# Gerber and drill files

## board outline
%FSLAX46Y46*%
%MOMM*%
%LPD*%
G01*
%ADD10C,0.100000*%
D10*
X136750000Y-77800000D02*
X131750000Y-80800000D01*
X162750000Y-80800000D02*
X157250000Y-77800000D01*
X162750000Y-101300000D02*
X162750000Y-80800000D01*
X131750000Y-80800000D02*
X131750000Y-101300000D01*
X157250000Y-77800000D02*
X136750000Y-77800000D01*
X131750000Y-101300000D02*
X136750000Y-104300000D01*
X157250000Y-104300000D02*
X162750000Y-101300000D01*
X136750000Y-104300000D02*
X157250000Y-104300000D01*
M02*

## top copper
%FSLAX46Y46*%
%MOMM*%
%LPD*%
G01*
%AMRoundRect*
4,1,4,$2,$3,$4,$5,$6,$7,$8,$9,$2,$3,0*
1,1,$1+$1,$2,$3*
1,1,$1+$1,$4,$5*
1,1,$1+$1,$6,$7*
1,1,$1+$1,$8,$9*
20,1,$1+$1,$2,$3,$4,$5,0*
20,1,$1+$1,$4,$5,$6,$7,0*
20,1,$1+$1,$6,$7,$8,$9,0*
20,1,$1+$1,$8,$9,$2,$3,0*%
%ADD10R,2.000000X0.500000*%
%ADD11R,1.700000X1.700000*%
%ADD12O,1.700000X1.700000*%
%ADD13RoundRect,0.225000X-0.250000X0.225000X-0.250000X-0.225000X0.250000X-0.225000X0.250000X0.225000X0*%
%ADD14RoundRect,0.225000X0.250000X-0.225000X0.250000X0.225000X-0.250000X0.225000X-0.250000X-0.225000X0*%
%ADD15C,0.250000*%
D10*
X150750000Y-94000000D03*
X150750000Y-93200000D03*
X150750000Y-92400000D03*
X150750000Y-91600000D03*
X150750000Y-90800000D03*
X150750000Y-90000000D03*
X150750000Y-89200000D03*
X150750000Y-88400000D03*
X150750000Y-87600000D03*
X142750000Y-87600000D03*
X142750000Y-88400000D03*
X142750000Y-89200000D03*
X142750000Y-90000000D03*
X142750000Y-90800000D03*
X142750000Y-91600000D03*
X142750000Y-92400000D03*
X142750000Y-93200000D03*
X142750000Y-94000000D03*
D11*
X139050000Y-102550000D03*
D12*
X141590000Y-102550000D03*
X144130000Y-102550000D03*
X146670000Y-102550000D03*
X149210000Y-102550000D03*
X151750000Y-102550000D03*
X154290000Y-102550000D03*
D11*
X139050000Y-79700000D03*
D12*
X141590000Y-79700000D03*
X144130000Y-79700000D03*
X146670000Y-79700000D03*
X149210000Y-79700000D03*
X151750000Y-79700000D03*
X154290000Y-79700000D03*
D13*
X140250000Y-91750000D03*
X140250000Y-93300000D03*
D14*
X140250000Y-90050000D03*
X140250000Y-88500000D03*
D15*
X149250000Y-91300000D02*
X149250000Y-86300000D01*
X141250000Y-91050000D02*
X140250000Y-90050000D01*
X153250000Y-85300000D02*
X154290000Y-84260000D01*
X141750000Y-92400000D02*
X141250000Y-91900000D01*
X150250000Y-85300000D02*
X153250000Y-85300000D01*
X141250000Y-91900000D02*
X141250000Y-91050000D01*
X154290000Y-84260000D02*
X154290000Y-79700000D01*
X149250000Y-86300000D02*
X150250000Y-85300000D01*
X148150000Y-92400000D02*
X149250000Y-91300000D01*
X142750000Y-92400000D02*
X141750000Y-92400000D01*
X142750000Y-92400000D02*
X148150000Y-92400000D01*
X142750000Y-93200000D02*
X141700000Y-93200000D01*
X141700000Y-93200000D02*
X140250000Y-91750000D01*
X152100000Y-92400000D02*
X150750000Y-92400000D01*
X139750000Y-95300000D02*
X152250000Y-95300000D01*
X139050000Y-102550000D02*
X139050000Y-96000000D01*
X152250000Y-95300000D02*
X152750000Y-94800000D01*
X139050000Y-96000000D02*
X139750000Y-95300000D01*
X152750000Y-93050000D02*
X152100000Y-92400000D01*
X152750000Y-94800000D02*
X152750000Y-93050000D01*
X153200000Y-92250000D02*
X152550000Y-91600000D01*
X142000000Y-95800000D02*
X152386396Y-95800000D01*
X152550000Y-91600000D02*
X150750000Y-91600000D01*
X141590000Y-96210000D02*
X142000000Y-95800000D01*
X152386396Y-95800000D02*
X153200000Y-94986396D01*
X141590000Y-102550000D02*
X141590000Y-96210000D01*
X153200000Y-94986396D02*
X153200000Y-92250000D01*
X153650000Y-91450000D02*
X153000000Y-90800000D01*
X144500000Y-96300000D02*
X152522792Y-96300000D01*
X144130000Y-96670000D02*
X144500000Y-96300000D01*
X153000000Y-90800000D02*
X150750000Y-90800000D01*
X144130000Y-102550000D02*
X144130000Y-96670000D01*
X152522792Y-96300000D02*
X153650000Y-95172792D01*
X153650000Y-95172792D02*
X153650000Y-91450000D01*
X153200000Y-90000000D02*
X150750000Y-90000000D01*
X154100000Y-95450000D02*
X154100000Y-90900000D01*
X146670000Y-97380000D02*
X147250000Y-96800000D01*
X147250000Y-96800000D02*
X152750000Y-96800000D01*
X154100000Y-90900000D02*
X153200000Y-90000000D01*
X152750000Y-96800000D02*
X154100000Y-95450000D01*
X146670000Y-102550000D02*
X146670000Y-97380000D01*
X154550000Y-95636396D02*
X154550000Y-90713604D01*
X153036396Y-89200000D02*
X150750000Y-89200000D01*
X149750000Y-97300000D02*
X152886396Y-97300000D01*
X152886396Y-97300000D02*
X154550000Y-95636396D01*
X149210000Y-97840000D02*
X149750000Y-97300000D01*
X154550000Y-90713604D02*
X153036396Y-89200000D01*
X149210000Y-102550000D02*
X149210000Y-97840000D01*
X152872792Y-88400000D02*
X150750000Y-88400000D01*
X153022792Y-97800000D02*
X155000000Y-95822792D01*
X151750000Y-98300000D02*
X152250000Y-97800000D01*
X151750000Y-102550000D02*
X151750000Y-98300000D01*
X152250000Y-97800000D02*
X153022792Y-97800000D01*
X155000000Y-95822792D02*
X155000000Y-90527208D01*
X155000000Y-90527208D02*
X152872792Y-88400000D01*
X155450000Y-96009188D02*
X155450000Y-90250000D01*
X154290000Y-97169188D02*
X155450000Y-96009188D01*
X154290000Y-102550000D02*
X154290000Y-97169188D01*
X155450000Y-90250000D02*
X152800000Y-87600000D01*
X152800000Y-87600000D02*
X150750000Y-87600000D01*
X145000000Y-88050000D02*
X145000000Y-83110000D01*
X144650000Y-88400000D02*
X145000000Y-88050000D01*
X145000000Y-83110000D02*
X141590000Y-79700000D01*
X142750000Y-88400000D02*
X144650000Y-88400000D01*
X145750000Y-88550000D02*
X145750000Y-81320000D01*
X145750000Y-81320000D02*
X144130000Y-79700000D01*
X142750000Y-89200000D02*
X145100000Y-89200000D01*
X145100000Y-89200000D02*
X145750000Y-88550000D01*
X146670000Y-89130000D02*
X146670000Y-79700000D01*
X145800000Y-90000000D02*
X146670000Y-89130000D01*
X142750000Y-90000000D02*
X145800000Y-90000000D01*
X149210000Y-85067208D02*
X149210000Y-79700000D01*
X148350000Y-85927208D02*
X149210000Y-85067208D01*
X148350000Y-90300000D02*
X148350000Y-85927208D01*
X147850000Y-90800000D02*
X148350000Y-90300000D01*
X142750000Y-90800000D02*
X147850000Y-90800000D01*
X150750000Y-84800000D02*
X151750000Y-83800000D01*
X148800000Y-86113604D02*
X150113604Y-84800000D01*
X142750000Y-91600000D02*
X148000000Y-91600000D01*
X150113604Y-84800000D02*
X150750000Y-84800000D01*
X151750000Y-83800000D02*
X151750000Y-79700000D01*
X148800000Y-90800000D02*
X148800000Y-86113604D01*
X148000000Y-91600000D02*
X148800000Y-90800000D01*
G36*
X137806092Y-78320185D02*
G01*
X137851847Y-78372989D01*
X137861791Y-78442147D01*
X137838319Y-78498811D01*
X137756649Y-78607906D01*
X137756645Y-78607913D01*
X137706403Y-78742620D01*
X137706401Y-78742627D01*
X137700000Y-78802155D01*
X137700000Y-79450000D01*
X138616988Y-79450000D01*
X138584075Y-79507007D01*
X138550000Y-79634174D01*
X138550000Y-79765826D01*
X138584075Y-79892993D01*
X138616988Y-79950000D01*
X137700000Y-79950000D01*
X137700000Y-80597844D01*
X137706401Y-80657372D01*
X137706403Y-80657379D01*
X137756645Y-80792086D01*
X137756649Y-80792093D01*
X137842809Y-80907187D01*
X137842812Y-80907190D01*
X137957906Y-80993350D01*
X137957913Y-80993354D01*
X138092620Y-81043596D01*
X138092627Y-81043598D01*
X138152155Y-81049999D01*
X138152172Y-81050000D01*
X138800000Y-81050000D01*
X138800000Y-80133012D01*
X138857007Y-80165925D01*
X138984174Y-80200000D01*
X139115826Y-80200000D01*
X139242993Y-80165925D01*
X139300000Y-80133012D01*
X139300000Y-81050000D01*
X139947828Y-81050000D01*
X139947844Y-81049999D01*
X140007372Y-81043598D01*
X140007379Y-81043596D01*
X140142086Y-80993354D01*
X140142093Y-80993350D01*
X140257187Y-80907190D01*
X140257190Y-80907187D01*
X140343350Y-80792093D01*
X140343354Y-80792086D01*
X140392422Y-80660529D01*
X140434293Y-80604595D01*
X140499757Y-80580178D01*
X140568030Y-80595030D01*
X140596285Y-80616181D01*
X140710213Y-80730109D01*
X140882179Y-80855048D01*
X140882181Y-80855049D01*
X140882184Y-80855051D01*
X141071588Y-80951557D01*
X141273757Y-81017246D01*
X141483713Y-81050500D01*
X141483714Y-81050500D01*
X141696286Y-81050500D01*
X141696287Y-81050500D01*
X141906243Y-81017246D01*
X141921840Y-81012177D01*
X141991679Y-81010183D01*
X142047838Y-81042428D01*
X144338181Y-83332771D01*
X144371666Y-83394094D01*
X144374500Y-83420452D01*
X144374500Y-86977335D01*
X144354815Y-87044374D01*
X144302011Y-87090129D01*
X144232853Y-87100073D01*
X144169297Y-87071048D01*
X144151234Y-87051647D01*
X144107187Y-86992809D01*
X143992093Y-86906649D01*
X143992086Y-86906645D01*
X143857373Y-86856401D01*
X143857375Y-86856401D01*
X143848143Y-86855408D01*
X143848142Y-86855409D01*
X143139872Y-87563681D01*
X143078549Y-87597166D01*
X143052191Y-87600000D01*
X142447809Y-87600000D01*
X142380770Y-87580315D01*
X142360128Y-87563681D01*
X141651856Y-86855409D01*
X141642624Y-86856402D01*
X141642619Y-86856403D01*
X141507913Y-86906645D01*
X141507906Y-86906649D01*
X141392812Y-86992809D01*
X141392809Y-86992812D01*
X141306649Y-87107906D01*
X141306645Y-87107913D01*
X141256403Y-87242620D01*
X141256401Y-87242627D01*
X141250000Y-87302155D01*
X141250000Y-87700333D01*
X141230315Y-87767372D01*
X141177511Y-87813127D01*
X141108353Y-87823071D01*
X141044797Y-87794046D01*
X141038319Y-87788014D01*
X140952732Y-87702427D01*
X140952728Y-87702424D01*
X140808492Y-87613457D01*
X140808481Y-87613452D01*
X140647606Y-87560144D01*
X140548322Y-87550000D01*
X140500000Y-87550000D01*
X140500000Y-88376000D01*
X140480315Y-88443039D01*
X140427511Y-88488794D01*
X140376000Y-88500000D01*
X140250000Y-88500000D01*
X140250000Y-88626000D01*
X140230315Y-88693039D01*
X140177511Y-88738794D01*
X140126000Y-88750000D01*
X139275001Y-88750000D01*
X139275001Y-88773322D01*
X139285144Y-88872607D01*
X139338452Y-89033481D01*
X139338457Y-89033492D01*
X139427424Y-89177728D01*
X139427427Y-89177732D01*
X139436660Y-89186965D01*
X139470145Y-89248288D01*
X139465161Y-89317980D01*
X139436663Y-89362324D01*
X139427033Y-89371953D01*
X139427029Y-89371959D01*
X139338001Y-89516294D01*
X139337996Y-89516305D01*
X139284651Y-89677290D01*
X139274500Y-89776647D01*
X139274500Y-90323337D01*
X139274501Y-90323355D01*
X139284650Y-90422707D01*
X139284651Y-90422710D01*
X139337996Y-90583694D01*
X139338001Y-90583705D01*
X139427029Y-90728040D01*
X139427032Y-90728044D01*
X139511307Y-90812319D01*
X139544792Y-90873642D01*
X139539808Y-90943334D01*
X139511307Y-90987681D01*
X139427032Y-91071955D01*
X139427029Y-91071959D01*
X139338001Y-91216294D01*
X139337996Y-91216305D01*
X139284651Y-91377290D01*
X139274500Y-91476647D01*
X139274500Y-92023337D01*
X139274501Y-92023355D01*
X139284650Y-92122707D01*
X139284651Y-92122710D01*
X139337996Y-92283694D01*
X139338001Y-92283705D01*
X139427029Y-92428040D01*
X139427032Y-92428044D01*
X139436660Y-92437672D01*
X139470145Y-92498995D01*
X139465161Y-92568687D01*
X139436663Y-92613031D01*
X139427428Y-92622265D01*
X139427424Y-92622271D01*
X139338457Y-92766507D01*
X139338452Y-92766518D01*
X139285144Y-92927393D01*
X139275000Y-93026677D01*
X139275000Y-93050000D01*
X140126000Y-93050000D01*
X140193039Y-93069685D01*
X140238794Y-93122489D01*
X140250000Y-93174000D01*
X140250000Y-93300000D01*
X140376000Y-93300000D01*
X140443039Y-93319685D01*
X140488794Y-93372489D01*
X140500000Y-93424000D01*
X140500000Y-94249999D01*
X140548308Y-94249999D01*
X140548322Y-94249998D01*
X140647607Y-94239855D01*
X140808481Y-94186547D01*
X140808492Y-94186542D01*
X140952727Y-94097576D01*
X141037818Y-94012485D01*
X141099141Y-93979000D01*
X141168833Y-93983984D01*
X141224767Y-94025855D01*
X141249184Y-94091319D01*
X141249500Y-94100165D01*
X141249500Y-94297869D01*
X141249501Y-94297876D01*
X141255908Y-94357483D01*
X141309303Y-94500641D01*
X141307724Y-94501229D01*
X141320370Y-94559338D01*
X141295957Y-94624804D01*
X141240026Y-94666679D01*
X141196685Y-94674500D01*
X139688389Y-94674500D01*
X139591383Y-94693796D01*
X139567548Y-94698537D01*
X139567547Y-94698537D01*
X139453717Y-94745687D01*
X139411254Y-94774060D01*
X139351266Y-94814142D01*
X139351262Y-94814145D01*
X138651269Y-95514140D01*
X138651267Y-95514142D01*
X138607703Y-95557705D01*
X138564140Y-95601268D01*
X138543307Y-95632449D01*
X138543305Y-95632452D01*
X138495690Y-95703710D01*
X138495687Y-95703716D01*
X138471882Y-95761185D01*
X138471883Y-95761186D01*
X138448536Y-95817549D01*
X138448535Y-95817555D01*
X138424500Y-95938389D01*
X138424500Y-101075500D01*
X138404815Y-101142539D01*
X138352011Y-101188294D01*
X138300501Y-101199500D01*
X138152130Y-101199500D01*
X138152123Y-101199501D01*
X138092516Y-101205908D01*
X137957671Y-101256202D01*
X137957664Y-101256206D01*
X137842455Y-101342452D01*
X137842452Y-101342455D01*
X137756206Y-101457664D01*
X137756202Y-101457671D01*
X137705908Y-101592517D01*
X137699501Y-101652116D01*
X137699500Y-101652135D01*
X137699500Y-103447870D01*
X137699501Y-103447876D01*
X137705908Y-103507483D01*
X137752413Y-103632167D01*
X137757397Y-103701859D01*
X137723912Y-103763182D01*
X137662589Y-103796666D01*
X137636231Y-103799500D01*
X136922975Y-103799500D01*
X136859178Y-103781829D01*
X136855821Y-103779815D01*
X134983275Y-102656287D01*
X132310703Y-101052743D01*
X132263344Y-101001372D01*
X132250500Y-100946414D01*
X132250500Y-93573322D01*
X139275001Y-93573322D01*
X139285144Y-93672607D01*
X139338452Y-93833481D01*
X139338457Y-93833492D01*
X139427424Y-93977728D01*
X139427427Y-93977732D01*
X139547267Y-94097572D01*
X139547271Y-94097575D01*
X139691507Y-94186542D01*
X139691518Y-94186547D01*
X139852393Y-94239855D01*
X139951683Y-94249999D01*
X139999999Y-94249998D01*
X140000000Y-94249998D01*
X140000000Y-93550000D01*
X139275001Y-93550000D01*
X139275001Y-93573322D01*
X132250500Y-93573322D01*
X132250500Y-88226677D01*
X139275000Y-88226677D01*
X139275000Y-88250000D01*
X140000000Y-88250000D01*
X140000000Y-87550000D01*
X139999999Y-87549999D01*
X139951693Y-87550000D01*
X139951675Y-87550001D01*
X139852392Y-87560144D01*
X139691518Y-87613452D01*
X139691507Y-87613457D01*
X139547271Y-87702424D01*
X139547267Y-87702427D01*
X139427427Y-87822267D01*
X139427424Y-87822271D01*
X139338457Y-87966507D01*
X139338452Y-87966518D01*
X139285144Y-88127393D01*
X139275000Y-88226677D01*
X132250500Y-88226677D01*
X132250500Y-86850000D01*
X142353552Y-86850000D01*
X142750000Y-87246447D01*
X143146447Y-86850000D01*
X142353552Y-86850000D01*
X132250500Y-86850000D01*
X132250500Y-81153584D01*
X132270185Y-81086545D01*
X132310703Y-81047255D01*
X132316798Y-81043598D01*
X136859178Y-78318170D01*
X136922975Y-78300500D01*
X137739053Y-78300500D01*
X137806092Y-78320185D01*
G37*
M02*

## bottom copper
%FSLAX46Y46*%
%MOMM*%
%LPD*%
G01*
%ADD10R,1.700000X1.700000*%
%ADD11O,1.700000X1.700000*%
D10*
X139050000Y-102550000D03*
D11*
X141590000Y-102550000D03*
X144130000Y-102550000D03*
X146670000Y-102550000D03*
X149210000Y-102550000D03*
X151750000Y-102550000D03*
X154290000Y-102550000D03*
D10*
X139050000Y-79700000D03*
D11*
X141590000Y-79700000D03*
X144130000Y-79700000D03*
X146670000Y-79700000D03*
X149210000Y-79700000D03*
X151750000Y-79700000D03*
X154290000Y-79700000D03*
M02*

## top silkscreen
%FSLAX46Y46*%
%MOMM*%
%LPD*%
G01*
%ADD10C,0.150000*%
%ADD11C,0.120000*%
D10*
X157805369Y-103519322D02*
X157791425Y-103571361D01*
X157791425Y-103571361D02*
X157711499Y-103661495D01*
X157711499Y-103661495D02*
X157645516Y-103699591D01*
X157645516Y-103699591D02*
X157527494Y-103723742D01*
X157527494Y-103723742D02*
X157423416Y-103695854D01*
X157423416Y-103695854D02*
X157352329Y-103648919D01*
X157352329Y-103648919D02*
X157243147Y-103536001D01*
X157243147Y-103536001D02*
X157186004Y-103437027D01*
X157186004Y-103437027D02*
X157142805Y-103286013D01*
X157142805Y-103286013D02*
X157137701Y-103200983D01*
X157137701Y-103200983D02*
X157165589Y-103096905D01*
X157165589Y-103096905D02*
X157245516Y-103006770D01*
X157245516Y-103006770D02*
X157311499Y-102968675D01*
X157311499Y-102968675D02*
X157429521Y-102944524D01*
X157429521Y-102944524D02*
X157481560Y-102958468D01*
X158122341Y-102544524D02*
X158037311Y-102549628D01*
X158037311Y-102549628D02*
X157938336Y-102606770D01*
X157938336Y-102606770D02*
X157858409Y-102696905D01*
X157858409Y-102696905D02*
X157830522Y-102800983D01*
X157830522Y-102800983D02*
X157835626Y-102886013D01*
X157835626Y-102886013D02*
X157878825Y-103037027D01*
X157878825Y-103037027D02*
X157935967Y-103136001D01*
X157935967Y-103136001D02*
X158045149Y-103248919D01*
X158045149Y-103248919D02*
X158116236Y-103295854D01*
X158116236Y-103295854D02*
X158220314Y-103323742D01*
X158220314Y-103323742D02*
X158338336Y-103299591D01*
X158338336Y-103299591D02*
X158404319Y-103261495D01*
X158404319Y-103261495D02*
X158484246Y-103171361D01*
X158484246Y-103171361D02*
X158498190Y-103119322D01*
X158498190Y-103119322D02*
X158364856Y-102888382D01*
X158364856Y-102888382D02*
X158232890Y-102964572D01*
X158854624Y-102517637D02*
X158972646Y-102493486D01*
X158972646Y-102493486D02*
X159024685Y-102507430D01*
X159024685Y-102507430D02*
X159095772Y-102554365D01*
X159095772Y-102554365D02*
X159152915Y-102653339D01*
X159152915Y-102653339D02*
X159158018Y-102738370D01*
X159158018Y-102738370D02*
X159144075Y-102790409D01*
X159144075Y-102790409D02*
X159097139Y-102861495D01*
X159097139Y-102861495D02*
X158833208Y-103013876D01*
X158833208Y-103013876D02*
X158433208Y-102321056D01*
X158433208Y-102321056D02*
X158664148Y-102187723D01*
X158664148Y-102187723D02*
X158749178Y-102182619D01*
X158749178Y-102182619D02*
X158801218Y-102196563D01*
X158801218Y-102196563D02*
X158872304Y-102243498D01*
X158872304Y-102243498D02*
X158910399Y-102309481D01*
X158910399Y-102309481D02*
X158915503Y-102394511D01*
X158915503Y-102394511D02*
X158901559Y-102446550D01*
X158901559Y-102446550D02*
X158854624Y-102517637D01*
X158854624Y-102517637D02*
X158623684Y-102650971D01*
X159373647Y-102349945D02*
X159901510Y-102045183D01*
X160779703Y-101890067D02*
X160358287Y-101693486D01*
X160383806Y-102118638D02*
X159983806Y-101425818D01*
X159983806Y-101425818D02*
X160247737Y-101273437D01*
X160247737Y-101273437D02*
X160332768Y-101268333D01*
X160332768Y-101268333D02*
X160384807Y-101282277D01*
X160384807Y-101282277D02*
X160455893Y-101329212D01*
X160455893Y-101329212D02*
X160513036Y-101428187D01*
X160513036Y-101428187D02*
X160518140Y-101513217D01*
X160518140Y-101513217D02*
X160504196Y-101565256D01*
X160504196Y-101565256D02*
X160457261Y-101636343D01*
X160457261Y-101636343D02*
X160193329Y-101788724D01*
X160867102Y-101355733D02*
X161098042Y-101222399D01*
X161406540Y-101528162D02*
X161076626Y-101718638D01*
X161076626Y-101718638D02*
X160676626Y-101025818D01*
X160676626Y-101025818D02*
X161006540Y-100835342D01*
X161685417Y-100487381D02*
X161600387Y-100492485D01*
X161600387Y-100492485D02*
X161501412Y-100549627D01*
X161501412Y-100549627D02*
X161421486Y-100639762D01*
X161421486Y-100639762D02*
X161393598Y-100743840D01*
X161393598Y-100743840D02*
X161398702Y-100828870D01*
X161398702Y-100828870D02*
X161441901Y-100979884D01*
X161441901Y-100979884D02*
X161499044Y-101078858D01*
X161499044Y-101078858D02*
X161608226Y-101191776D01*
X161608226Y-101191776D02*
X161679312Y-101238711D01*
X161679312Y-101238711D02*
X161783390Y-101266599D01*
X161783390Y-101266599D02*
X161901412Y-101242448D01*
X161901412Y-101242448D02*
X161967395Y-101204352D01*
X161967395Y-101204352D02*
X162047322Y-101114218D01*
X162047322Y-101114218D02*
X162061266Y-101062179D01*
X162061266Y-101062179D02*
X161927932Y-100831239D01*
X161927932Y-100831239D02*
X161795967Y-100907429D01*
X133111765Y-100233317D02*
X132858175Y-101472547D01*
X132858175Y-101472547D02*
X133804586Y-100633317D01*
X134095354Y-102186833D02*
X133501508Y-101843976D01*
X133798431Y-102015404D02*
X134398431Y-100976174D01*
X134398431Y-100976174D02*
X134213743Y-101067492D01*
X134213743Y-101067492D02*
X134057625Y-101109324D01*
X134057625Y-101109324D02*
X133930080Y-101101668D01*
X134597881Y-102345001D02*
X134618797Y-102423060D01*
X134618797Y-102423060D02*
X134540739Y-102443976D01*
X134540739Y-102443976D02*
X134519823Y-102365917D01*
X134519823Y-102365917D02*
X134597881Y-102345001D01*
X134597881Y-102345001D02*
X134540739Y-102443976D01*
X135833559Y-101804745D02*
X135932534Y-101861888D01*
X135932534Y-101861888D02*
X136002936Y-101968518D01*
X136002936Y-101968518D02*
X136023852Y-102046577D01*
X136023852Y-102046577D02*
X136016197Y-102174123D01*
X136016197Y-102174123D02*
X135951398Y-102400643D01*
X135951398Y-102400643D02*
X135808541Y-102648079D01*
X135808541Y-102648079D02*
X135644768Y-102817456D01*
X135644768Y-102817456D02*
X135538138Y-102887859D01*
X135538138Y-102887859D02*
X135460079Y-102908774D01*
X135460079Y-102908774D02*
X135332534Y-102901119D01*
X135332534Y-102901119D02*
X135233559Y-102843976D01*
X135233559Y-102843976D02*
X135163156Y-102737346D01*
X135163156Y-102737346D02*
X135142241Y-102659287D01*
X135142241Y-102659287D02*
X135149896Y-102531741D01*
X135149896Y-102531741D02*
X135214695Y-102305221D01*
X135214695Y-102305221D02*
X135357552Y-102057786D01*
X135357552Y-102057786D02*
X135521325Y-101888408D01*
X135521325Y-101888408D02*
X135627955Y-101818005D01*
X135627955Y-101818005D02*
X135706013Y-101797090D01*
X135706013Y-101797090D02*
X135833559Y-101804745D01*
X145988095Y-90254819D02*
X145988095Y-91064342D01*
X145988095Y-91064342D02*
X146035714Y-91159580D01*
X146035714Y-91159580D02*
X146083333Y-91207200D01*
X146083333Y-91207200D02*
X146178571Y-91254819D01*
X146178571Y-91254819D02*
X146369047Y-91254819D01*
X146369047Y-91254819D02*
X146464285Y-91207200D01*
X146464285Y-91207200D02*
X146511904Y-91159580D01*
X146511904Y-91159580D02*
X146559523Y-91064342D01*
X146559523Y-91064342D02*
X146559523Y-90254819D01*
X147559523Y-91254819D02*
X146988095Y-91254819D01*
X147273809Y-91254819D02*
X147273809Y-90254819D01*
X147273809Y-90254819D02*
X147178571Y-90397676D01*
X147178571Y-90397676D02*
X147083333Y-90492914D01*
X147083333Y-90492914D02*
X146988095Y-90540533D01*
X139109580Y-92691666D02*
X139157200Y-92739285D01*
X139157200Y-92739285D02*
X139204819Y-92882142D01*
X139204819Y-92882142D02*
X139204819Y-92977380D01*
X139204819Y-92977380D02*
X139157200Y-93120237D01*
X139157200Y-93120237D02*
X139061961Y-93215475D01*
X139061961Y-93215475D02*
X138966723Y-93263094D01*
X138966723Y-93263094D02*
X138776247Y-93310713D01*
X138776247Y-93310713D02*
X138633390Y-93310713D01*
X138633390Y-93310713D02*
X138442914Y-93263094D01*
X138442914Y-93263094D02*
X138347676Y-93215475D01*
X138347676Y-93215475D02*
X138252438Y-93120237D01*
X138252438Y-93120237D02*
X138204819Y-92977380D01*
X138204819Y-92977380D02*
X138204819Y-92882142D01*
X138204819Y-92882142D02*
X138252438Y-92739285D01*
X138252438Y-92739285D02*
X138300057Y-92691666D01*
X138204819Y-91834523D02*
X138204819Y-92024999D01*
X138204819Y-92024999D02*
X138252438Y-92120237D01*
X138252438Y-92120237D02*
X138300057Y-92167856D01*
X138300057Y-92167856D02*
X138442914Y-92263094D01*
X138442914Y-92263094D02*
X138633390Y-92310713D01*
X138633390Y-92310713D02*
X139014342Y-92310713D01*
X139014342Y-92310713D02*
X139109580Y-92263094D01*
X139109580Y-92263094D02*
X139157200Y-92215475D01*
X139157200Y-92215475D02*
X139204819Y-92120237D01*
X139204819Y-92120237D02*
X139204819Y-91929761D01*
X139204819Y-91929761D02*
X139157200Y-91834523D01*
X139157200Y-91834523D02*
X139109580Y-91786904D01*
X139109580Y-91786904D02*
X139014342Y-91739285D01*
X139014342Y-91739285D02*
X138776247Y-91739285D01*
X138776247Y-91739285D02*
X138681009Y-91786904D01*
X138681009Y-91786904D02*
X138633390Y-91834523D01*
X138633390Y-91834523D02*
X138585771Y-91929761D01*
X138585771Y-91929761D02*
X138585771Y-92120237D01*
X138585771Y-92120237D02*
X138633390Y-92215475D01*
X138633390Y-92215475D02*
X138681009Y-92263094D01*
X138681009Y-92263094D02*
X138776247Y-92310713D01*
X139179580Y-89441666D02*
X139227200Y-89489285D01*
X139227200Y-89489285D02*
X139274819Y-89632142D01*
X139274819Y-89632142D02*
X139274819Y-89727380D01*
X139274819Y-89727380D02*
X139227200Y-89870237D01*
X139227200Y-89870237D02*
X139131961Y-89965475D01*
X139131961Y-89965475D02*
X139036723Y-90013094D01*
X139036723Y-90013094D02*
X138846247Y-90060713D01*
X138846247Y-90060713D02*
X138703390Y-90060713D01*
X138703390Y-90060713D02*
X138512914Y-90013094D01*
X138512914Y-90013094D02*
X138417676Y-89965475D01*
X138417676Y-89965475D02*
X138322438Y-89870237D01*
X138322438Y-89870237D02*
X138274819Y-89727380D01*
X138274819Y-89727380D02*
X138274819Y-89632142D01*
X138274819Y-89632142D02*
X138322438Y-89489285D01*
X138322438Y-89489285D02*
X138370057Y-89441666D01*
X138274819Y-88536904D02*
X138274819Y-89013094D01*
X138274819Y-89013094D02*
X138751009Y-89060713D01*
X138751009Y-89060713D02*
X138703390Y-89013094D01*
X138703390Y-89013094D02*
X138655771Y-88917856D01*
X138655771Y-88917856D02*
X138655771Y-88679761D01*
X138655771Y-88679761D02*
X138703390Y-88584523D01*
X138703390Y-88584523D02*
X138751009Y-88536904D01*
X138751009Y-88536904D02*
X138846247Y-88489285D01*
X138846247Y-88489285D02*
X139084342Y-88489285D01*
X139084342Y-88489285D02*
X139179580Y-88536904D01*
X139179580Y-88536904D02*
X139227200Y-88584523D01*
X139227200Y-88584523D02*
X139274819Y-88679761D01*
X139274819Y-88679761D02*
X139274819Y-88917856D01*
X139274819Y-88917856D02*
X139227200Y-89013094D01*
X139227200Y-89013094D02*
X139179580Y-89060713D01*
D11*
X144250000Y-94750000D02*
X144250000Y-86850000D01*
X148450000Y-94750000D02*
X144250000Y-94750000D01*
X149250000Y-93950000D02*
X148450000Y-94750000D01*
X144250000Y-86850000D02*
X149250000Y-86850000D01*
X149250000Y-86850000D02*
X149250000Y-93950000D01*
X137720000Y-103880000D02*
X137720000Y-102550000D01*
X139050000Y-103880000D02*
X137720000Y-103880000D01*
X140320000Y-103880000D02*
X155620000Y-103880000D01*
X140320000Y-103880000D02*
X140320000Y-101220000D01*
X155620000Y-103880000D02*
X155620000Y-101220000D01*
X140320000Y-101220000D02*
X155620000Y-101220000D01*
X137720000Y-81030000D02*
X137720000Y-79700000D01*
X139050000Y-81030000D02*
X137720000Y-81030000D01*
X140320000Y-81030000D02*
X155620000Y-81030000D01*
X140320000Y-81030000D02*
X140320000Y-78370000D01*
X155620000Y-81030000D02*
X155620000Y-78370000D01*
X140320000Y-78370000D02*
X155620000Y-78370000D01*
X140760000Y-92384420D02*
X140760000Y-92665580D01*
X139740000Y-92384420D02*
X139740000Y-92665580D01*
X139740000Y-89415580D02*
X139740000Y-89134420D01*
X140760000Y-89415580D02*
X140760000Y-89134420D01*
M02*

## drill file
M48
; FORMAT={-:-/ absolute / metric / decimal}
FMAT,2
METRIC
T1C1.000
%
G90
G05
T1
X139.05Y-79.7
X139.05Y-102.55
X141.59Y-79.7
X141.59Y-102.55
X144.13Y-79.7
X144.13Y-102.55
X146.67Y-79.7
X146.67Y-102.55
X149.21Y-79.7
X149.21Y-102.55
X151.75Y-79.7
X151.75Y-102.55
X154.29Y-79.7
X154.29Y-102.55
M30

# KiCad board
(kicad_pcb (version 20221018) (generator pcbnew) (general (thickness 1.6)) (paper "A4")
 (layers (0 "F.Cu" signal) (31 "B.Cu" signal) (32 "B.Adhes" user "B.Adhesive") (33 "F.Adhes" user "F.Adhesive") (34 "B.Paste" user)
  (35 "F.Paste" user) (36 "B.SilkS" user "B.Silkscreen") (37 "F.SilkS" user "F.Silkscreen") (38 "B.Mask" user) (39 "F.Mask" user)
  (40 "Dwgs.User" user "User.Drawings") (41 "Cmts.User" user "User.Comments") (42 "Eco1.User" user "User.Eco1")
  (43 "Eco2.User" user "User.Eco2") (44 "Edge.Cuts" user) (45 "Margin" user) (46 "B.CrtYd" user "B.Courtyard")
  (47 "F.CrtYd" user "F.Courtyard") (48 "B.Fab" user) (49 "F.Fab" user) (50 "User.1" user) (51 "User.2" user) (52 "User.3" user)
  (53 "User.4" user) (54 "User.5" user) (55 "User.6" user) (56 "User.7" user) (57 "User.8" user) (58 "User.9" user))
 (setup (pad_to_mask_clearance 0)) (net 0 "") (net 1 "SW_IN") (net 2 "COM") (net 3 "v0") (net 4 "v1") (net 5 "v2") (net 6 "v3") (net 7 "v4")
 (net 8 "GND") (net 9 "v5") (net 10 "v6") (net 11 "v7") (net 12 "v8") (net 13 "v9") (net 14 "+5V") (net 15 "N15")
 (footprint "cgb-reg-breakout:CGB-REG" (layer "F.Cu") (at 146.75 90.8 90)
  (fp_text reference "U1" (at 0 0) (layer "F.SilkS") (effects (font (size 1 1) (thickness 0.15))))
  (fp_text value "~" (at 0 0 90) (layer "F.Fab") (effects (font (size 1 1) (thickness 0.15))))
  (fp_line (start -3.95 -2.5) (end 3.95 -2.5) (stroke (width 0.12) (type default)) (layer "F.SilkS"))
  (fp_line (start -3.95 1.7) (end -3.95 -2.5) (stroke (width 0.12) (type default)) (layer "F.SilkS"))
  (fp_line (start -3.15 2.5) (end -3.95 1.7) (stroke (width 0.12) (type default)) (layer "F.SilkS"))
  (fp_line (start 3.95 -2.5) (end 3.95 2.5) (stroke (width 0.12) (type default)) (layer "F.SilkS"))
  (fp_line (start 3.95 2.5) (end -3.15 2.5) (stroke (width 0.12) (type default)) (layer "F.SilkS"))
  (pad "1" smd rect (at -3.2 4 90) (size 0.5 2) (layers "F.Cu" "F.Paste" "F.Mask") (thermal_bridge_angle 45))
  (pad "2" smd rect (at -2.4 4 90) (size 0.5 2) (layers "F.Cu" "F.Paste" "F.Mask") (thermal_bridge_angle 45))
  (pad "3" smd rect (at -1.6 4 90) (size 0.5 2) (layers "F.Cu" "F.Paste" "F.Mask") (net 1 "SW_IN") (thermal_bridge_angle 45))
  (pad "4" smd rect (at -0.8 4 90) (size 0.5 2) (layers "F.Cu" "F.Paste" "F.Mask") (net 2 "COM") (thermal_bridge_angle 45))
  (pad "5" smd rect (at 0 4 90) (size 0.5 2) (layers "F.Cu" "F.Paste" "F.Mask") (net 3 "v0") (thermal_bridge_angle 45))
  (pad "6" smd rect (at 0.8 4 90) (size 0.5 2) (layers "F.Cu" "F.Paste" "F.Mask") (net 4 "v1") (thermal_bridge_angle 45))
  (pad "7" smd rect (at 1.6 4 90) (size 0.5 2) (layers "F.Cu" "F.Paste" "F.Mask") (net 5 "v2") (thermal_bridge_angle 45))
  (pad "8" smd rect (at 2.4 4 90) (size 0.5 2) (layers "F.Cu" "F.Paste" "F.Mask") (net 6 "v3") (thermal_bridge_angle 45))
  (pad "9" smd rect (at 3.2 4 90) (size 0.5 2) (layers "F.Cu" "F.Paste" "F.Mask") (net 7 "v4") (thermal_bridge_angle 45))
  (pad "10" smd rect (at 3.2 -4 90) (size 0.5 2) (layers "F.Cu" "F.Paste" "F.Mask") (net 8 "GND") (thermal_bridge_angle 45))
  (pad "11" smd rect (at 2.4 -4 90) (size 0.5 2) (layers "F.Cu" "F.Paste" "F.Mask") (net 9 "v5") (thermal_bridge_angle 45))
  (pad "12" smd rect (at 1.6 -4 90) (size 0.5 2) (layers "F.Cu" "F.Paste" "F.Mask") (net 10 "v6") (thermal_bridge_angle 45))
  (pad "13" smd rect (at 0.8 -4 90) (size 0.5 2) (layers "F.Cu" "F.Paste" "F.Mask") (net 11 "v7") (thermal_bridge_angle 45))
  (pad "14" smd rect (at 0 -4 90) (size 0.5 2) (layers "F.Cu" "F.Paste" "F.Mask") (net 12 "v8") (thermal_bridge_angle 45))
  (pad "15" smd rect (at -0.8 -4 90) (size 0.5 2) (layers "F.Cu" "F.Paste" "F.Mask") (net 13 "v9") (thermal_bridge_angle 45))
  (pad "16" smd rect (at -1.6 -4 90) (size 0.5 2) (layers "F.Cu" "F.Paste" "F.Mask") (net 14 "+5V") (thermal_bridge_angle 45))
  (pad "17" smd rect (at -2.4 -4 90) (size 0.5 2) (layers "F.Cu" "F.Paste" "F.Mask") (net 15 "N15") (thermal_bridge_angle 45))
  (pad "18" smd rect (at -3.2 -4 90) (size 0.5 2) (layers "F.Cu" "F.Paste" "F.Mask") (thermal_bridge_angle 45)))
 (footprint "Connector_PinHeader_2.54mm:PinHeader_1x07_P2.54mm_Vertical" (layer "F.Cu") (at 139.05 102.55 90)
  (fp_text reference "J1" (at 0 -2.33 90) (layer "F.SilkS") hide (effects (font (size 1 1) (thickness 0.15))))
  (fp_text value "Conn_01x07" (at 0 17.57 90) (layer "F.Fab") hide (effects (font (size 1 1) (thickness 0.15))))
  (fp_line (start -1.33 -1.33) (end 0 -1.33) (stroke (width 0.12) (type solid)) (layer "F.SilkS"))
  (fp_line (start -1.33 0) (end -1.33 -1.33) (stroke (width 0.12) (type solid)) (layer "F.SilkS"))
  (fp_line (start -1.33 1.27) (end -1.33 16.57) (stroke (width 0.12) (type solid)) (layer "F.SilkS"))
  (fp_line (start -1.33 1.27) (end 1.33 1.27) (stroke (width 0.12) (type solid)) (layer "F.SilkS"))
  (fp_line (start -1.33 16.57) (end 1.33 16.57) (stroke (width 0.12) (type solid)) (layer "F.SilkS"))
  (fp_line (start 1.33 1.27) (end 1.33 16.57) (stroke (width 0.12) (type solid)) (layer "F.SilkS"))
  (pad "1" thru_hole rect (at 0 0 90) (size 1.7 1.7) (drill 1) (layers "*.Cu" "*.Mask") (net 1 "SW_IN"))
  (pad "2" thru_hole oval (at 0 2.54 90) (size 1.7 1.7) (drill 1) (layers "*.Cu" "*.Mask") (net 2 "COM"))
  (pad "3" thru_hole oval (at 0 5.08 90) (size 1.7 1.7) (drill 1) (layers "*.Cu" "*.Mask") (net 3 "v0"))
  (pad "4" thru_hole oval (at 0 7.62 90) (size 1.7 1.7) (drill 1) (layers "*.Cu" "*.Mask") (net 4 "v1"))
  (pad "5" thru_hole oval (at 0 10.16 90) (size 1.7 1.7) (drill 1) (layers "*.Cu" "*.Mask") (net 5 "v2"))
  (pad "6" thru_hole oval (at 0 12.7 90) (size 1.7 1.7) (drill 1) (layers "*.Cu" "*.Mask") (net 6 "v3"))
  (pad "7" thru_hole oval (at 0 15.24 90) (size 1.7 1.7) (drill 1) (layers "*.Cu" "*.Mask") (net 7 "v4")))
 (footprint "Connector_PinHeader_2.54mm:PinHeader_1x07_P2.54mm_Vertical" (layer "F.Cu") (at 139.05 79.7 90)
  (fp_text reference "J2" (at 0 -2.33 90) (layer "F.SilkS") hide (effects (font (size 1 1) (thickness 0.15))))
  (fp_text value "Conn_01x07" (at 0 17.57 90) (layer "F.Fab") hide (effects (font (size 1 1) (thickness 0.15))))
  (fp_line (start -1.33 -1.33) (end 0 -1.33) (stroke (width 0.12) (type solid)) (layer "F.SilkS"))
  (fp_line (start -1.33 0) (end -1.33 -1.33) (stroke (width 0.12) (type solid)) (layer "F.SilkS"))
  (fp_line (start -1.33 1.27) (end -1.33 16.57) (stroke (width 0.12) (type solid)) (layer "F.SilkS"))
  (fp_line (start -1.33 1.27) (end 1.33 1.27) (stroke (width 0.12) (type solid)) (layer "F.SilkS"))
  (fp_line (start -1.33 16.57) (end 1.33 16.57) (stroke (width 0.12) (type solid)) (layer "F.SilkS"))
  (fp_line (start 1.33 1.27) (end 1.33 16.57) (stroke (width 0.12) (type solid)) (layer "F.SilkS"))
  (pad "1" thru_hole rect (at 0 0 90) (size 1.7 1.7) (drill 1) (layers "*.Cu" "*.Mask") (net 8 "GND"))
  (pad "2" thru_hole oval (at 0 2.54 90) (size 1.7 1.7) (drill 1) (layers "*.Cu" "*.Mask") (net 9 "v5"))
  (pad "3" thru_hole oval (at 0 5.08 90) (size 1.7 1.7) (drill 1) (layers "*.Cu" "*.Mask") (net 10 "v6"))
  (pad "4" thru_hole oval (at 0 7.62 90) (size 1.7 1.7) (drill 1) (layers "*.Cu" "*.Mask") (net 11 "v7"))
  (pad "5" thru_hole oval (at 0 10.16 90) (size 1.7 1.7) (drill 1) (layers "*.Cu" "*.Mask") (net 12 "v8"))
  (pad "6" thru_hole oval (at 0 12.7 90) (size 1.7 1.7) (drill 1) (layers "*.Cu" "*.Mask") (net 13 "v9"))
  (pad "7" thru_hole oval (at 0 15.24 90) (size 1.7 1.7) (drill 1) (layers "*.Cu" "*.Mask") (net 14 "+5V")))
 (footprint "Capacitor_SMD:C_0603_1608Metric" (layer "F.Cu") (at 140.25 92.525 -90)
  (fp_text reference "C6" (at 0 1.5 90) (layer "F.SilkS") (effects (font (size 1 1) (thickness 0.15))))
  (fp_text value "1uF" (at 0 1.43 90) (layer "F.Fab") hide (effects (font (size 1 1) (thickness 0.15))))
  (fp_line (start -0.14058 -0.51) (end 0.14058 -0.51) (stroke (width 0.12) (type solid)) (layer "F.SilkS"))
  (fp_line (start -0.14058 0.51) (end 0.14058 0.51) (stroke (width 0.12) (type solid)) (layer "F.SilkS"))
  (pad "1" smd roundrect (at -0.775 0 270) (size 0.9 0.95) (layers "F.Cu" "F.Paste" "F.Mask") (roundrect_rratio 0.25) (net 15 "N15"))
  (pad "2" smd roundrect (at 0.775 0 270) (size 0.9 0.95) (layers "F.Cu" "F.Paste" "F.Mask") (roundrect_rratio 0.25) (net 8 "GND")))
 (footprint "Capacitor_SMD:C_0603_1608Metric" (layer "F.Cu") (at 140.25 89.275 90)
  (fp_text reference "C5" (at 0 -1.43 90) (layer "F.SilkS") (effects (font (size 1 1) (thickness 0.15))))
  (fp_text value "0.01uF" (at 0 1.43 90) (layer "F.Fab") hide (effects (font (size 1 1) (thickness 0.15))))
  (fp_line (start -0.14058 -0.51) (end 0.14058 -0.51) (stroke (width 0.12) (type solid)) (layer "F.SilkS"))
  (fp_line (start -0.14058 0.51) (end 0.14058 0.51) (stroke (width 0.12) (type solid)) (layer "F.SilkS"))
  (pad "1" smd roundrect (at -0.775 0 90) (size 0.9 0.95) (layers "F.Cu" "F.Paste" "F.Mask") (roundrect_rratio 0.25) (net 14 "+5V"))
  (pad "2" smd roundrect (at 0.775 0 90) (size 0.9 0.95) (layers "F.Cu" "F.Paste" "F.Mask") (roundrect_rratio 0.25) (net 8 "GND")))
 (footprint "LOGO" (layer "B.Cu") (at 146.75 90.8 -90)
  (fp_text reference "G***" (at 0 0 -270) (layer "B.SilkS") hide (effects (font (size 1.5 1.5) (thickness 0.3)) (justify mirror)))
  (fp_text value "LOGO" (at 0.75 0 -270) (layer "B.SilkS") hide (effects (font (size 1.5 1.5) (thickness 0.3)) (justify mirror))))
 (gr_line (start 136.75 77.8) (end 131.75 80.8) (stroke (width 0.1) (type default)) (layer "Edge.Cuts"))
 (gr_line (start 162.75 80.8) (end 157.25 77.8) (stroke (width 0.1) (type default)) (layer "Edge.Cuts"))
 (gr_line (start 162.75 101.3) (end 162.75 80.8) (stroke (width 0.1) (type default)) (layer "Edge.Cuts"))
 (gr_line (start 131.75 80.8) (end 131.75 101.3) (stroke (width 0.1) (type default)) (layer "Edge.Cuts"))
 (gr_line (start 157.25 77.8) (end 136.75 77.8) (stroke (width 0.1) (type default)) (layer "Edge.Cuts"))
 (gr_line (start 131.75 101.3) (end 136.75 104.3) (stroke (width 0.1) (type default)) (layer "Edge.Cuts"))
 (gr_line (start 157.25 104.3) (end 162.75 101.3) (stroke (width 0.1) (type default)) (layer "Edge.Cuts"))
 (gr_line (start 136.75 104.3) (end 157.25 104.3) (stroke (width 0.1) (type default)) (layer "Edge.Cuts"))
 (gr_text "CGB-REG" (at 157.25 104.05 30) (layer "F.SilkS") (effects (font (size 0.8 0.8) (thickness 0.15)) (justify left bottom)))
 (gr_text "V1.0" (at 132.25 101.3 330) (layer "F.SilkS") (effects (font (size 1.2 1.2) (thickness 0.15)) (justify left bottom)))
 (segment (start 149.25 91.3) (end 149.25 86.3) (width 0.25) (layer "F.Cu") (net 14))
 (segment (start 141.25 91.05) (end 140.25 90.05) (width 0.25) (layer "F.Cu") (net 14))
 (segment (start 153.25 85.3) (end 154.29 84.26) (width 0.25) (layer "F.Cu") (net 14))
 (segment (start 141.75 92.4) (end 141.25 91.9) (width 0.25) (layer "F.Cu") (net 14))
 (segment (start 150.25 85.3) (end 153.25 85.3) (width 0.25) (layer "F.Cu") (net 14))
 (segment (start 141.25 91.9) (end 141.25 91.05) (width 0.25) (layer "F.Cu") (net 14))
 (segment (start 154.29 84.26) (end 154.29 79.7) (width 0.25) (layer "F.Cu") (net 14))
 (segment (start 149.25 86.3) (end 150.25 85.3) (width 0.25) (layer "F.Cu") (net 14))
 (segment (start 148.15 92.4) (end 149.25 91.3) (width 0.25) (layer "F.Cu") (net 14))
 (segment (start 142.75 92.4) (end 141.75 92.4) (width 0.25) (layer "F.Cu") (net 14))
 (segment (start 142.75 92.4) (end 148.15 92.4) (width 0.25) (layer "F.Cu") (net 14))
 (segment (start 142.75 93.2) (end 141.7 93.2) (width 0.25) (layer "F.Cu") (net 15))
 (segment (start 141.7 93.2) (end 140.25 91.75) (width 0.25) (layer "F.Cu") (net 15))
 (segment (start 152.1 92.4) (end 150.75 92.4) (width 0.25) (layer "F.Cu") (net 1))
 (segment (start 139.75 95.3) (end 152.25 95.3) (width 0.25) (layer "F.Cu") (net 1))
 (segment (start 139.05 102.55) (end 139.05 96) (width 0.25) (layer "F.Cu") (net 1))
 (segment (start 152.25 95.3) (end 152.75 94.8) (width 0.25) (layer "F.Cu") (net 1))
 (segment (start 139.05 96) (end 139.75 95.3) (width 0.25) (layer "F.Cu") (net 1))
 (segment (start 152.75 93.05) (end 152.1 92.4) (width 0.25) (layer "F.Cu") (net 1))
 (segment (start 152.75 94.8) (end 152.75 93.05) (width 0.25) (layer "F.Cu") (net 1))
 (segment (start 153.2 92.25) (end 152.55 91.6) (width 0.25) (layer "F.Cu") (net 2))
 (segment (start 142 95.8) (end 152.386396 95.8) (width 0.25) (layer "F.Cu") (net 2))
 (segment (start 152.55 91.6) (end 150.75 91.6) (width 0.25) (layer "F.Cu") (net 2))
 (segment (start 141.59 96.21) (end 142 95.8) (width 0.25) (layer "F.Cu") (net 2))
 (segment (start 152.386396 95.8) (end 153.2 94.986396) (width 0.25) (layer "F.Cu") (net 2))
 (segment (start 141.59 102.55) (end 141.59 96.21) (width 0.25) (layer "F.Cu") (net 2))
 (segment (start 153.2 94.986396) (end 153.2 92.25) (width 0.25) (layer "F.Cu") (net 2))
 (segment (start 153.65 91.45) (end 153 90.8) (width 0.25) (layer "F.Cu") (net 3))
 (segment (start 144.5 96.3) (end 152.522792 96.3) (width 0.25) (layer "F.Cu") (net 3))
 (segment (start 144.13 96.67) (end 144.5 96.3) (width 0.25) (layer "F.Cu") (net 3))
 (segment (start 153 90.8) (end 150.75 90.8) (width 0.25) (layer "F.Cu") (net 3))
 (segment (start 144.13 102.55) (end 144.13 96.67) (width 0.25) (layer "F.Cu") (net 3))
 (segment (start 152.522792 96.3) (end 153.65 95.172792) (width 0.25) (layer "F.Cu") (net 3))
 (segment (start 153.65 95.172792) (end 153.65 91.45) (width 0.25) (layer "F.Cu") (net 3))
 (segment (start 153.2 90) (end 150.75 90) (width 0.25) (layer "F.Cu") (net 4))
 (segment (start 154.1 95.45) (end 154.1 90.9) (width 0.25) (layer "F.Cu") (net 4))
 (segment (start 146.67 97.38) (end 147.25 96.8) (width 0.25) (layer "F.Cu") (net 4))
 (segment (start 147.25 96.8) (end 152.75 96.8) (width 0.25) (layer "F.Cu") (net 4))
 (segment (start 154.1 90.9) (end 153.2 90) (width 0.25) (layer "F.Cu") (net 4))
 (segment (start 152.75 96.8) (end 154.1 95.45) (width 0.25) (layer "F.Cu") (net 4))
 (segment (start 146.67 102.55) (end 146.67 97.38) (width 0.25) (layer "F.Cu") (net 4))
 (segment (start 154.55 95.636396) (end 154.55 90.713604) (width 0.25) (layer "F.Cu") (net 5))
 (segment (start 153.036396 89.2) (end 150.75 89.2) (width 0.25) (layer "F.Cu") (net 5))
 (segment (start 149.75 97.3) (end 152.886396 97.3) (width 0.25) (layer "F.Cu") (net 5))
 (segment (start 152.886396 97.3) (end 154.55 95.636396) (width 0.25) (layer "F.Cu") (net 5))
 (segment (start 149.21 97.84) (end 149.75 97.3) (width 0.25) (layer "F.Cu") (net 5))
 (segment (start 154.55 90.713604) (end 153.036396 89.2) (width 0.25) (layer "F.Cu") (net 5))
 (segment (start 149.21 102.55) (end 149.21 97.84) (width 0.25) (layer "F.Cu") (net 5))
 (segment (start 152.872792 88.4) (end 150.75 88.4) (width 0.25) (layer "F.Cu") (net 6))
 (segment (start 153.022792 97.8) (end 155 95.822792) (width 0.25) (layer "F.Cu") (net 6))
 (segment (start 151.75 98.3) (end 152.25 97.8) (width 0.25) (layer "F.Cu") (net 6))
 (segment (start 151.75 102.55) (end 151.75 98.3) (width 0.25) (layer "F.Cu") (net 6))
 (segment (start 152.25 97.8) (end 153.022792 97.8) (width 0.25) (layer "F.Cu") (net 6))
 (segment (start 155 95.822792) (end 155 90.527208) (width 0.25) (layer "F.Cu") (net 6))
 (segment (start 155 90.527208) (end 152.872792 88.4) (width 0.25) (layer "F.Cu") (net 6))
 (segment (start 155.45 96.009188) (end 155.45 90.25) (width 0.25) (layer "F.Cu") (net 7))
 (segment (start 154.29 97.169188) (end 155.45 96.009188) (width 0.25) (layer "F.Cu") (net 7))
 (segment (start 154.29 102.55) (end 154.29 97.169188) (width 0.25) (layer "F.Cu") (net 7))
 (segment (start 155.45 90.25) (end 152.8 87.6) (width 0.25) (layer "F.Cu") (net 7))
 (segment (start 152.8 87.6) (end 150.75 87.6) (width 0.25) (layer "F.Cu") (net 7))
 (segment (start 145 88.05) (end 145 83.11) (width 0.25) (layer "F.Cu") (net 9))
 (segment (start 144.65 88.4) (end 145 88.05) (width 0.25) (layer "F.Cu") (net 9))
 (segment (start 145 83.11) (end 141.59 79.7) (width 0.25) (layer "F.Cu") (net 9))
 (segment (start 142.75 88.4) (end 144.65 88.4) (width 0.25) (layer "F.Cu") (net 9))
 (segment (start 145.75 88.55) (end 145.75 81.32) (width 0.25) (layer "F.Cu") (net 10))
 (segment (start 145.75 81.32) (end 144.13 79.7) (width 0.25) (layer "F.Cu") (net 10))
 (segment (start 142.75 89.2) (end 145.1 89.2) (width 0.25) (layer "F.Cu") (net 10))
 (segment (start 145.1 89.2) (end 145.75 88.55) (width 0.25) (layer "F.Cu") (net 10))
 (segment (start 146.67 89.13) (end 146.67 79.7) (width 0.25) (layer "F.Cu") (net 11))
 (segment (start 145.8 90) (end 146.67 89.13) (width 0.25) (layer "F.Cu") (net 11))
 (segment (start 142.75 90) (end 145.8 90) (width 0.25) (layer "F.Cu") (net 11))
 (segment (start 149.21 85.067208) (end 149.21 79.7) (width 0.25) (layer "F.Cu") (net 12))
 (segment (start 148.35 85.927208) (end 149.21 85.067208) (width 0.25) (layer "F.Cu") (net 12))
 (segment (start 148.35 90.3) (end 148.35 85.927208) (width 0.25) (layer "F.Cu") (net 12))
 (segment (start 147.85 90.8) (end 148.35 90.3) (width 0.25) (layer "F.Cu") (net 12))
 (segment (start 142.75 90.8) (end 147.85 90.8) (width 0.25) (layer "F.Cu") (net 12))
 (segment (start 150.75 84.8) (end 151.75 83.8) (width 0.25) (layer "F.Cu") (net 13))
 (segment (start 148.8 86.113604) (end 150.113604 84.8) (width 0.25) (layer "F.Cu") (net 13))
 (segment (start 142.75 91.6) (end 148 91.6) (width 0.25) (layer "F.Cu") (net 13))
 (segment (start 150.113604 84.8) (end 150.75 84.8) (width 0.25) (layer "F.Cu") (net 13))
 (segment (start 151.75 83.8) (end 151.75 79.7) (width 0.25) (layer "F.Cu") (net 13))
 (segment (start 148.8 90.8) (end 148.8 86.113604) (width 0.25) (layer "F.Cu") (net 13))
 (segment (start 148 91.6) (end 148.8 90.8) (width 0.25) (layer "F.Cu") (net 13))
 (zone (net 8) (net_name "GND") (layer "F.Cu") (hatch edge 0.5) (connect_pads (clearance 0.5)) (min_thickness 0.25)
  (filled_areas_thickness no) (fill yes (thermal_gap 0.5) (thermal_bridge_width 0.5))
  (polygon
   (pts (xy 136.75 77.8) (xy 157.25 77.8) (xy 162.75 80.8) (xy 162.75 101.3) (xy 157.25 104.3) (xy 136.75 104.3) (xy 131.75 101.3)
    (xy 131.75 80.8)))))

